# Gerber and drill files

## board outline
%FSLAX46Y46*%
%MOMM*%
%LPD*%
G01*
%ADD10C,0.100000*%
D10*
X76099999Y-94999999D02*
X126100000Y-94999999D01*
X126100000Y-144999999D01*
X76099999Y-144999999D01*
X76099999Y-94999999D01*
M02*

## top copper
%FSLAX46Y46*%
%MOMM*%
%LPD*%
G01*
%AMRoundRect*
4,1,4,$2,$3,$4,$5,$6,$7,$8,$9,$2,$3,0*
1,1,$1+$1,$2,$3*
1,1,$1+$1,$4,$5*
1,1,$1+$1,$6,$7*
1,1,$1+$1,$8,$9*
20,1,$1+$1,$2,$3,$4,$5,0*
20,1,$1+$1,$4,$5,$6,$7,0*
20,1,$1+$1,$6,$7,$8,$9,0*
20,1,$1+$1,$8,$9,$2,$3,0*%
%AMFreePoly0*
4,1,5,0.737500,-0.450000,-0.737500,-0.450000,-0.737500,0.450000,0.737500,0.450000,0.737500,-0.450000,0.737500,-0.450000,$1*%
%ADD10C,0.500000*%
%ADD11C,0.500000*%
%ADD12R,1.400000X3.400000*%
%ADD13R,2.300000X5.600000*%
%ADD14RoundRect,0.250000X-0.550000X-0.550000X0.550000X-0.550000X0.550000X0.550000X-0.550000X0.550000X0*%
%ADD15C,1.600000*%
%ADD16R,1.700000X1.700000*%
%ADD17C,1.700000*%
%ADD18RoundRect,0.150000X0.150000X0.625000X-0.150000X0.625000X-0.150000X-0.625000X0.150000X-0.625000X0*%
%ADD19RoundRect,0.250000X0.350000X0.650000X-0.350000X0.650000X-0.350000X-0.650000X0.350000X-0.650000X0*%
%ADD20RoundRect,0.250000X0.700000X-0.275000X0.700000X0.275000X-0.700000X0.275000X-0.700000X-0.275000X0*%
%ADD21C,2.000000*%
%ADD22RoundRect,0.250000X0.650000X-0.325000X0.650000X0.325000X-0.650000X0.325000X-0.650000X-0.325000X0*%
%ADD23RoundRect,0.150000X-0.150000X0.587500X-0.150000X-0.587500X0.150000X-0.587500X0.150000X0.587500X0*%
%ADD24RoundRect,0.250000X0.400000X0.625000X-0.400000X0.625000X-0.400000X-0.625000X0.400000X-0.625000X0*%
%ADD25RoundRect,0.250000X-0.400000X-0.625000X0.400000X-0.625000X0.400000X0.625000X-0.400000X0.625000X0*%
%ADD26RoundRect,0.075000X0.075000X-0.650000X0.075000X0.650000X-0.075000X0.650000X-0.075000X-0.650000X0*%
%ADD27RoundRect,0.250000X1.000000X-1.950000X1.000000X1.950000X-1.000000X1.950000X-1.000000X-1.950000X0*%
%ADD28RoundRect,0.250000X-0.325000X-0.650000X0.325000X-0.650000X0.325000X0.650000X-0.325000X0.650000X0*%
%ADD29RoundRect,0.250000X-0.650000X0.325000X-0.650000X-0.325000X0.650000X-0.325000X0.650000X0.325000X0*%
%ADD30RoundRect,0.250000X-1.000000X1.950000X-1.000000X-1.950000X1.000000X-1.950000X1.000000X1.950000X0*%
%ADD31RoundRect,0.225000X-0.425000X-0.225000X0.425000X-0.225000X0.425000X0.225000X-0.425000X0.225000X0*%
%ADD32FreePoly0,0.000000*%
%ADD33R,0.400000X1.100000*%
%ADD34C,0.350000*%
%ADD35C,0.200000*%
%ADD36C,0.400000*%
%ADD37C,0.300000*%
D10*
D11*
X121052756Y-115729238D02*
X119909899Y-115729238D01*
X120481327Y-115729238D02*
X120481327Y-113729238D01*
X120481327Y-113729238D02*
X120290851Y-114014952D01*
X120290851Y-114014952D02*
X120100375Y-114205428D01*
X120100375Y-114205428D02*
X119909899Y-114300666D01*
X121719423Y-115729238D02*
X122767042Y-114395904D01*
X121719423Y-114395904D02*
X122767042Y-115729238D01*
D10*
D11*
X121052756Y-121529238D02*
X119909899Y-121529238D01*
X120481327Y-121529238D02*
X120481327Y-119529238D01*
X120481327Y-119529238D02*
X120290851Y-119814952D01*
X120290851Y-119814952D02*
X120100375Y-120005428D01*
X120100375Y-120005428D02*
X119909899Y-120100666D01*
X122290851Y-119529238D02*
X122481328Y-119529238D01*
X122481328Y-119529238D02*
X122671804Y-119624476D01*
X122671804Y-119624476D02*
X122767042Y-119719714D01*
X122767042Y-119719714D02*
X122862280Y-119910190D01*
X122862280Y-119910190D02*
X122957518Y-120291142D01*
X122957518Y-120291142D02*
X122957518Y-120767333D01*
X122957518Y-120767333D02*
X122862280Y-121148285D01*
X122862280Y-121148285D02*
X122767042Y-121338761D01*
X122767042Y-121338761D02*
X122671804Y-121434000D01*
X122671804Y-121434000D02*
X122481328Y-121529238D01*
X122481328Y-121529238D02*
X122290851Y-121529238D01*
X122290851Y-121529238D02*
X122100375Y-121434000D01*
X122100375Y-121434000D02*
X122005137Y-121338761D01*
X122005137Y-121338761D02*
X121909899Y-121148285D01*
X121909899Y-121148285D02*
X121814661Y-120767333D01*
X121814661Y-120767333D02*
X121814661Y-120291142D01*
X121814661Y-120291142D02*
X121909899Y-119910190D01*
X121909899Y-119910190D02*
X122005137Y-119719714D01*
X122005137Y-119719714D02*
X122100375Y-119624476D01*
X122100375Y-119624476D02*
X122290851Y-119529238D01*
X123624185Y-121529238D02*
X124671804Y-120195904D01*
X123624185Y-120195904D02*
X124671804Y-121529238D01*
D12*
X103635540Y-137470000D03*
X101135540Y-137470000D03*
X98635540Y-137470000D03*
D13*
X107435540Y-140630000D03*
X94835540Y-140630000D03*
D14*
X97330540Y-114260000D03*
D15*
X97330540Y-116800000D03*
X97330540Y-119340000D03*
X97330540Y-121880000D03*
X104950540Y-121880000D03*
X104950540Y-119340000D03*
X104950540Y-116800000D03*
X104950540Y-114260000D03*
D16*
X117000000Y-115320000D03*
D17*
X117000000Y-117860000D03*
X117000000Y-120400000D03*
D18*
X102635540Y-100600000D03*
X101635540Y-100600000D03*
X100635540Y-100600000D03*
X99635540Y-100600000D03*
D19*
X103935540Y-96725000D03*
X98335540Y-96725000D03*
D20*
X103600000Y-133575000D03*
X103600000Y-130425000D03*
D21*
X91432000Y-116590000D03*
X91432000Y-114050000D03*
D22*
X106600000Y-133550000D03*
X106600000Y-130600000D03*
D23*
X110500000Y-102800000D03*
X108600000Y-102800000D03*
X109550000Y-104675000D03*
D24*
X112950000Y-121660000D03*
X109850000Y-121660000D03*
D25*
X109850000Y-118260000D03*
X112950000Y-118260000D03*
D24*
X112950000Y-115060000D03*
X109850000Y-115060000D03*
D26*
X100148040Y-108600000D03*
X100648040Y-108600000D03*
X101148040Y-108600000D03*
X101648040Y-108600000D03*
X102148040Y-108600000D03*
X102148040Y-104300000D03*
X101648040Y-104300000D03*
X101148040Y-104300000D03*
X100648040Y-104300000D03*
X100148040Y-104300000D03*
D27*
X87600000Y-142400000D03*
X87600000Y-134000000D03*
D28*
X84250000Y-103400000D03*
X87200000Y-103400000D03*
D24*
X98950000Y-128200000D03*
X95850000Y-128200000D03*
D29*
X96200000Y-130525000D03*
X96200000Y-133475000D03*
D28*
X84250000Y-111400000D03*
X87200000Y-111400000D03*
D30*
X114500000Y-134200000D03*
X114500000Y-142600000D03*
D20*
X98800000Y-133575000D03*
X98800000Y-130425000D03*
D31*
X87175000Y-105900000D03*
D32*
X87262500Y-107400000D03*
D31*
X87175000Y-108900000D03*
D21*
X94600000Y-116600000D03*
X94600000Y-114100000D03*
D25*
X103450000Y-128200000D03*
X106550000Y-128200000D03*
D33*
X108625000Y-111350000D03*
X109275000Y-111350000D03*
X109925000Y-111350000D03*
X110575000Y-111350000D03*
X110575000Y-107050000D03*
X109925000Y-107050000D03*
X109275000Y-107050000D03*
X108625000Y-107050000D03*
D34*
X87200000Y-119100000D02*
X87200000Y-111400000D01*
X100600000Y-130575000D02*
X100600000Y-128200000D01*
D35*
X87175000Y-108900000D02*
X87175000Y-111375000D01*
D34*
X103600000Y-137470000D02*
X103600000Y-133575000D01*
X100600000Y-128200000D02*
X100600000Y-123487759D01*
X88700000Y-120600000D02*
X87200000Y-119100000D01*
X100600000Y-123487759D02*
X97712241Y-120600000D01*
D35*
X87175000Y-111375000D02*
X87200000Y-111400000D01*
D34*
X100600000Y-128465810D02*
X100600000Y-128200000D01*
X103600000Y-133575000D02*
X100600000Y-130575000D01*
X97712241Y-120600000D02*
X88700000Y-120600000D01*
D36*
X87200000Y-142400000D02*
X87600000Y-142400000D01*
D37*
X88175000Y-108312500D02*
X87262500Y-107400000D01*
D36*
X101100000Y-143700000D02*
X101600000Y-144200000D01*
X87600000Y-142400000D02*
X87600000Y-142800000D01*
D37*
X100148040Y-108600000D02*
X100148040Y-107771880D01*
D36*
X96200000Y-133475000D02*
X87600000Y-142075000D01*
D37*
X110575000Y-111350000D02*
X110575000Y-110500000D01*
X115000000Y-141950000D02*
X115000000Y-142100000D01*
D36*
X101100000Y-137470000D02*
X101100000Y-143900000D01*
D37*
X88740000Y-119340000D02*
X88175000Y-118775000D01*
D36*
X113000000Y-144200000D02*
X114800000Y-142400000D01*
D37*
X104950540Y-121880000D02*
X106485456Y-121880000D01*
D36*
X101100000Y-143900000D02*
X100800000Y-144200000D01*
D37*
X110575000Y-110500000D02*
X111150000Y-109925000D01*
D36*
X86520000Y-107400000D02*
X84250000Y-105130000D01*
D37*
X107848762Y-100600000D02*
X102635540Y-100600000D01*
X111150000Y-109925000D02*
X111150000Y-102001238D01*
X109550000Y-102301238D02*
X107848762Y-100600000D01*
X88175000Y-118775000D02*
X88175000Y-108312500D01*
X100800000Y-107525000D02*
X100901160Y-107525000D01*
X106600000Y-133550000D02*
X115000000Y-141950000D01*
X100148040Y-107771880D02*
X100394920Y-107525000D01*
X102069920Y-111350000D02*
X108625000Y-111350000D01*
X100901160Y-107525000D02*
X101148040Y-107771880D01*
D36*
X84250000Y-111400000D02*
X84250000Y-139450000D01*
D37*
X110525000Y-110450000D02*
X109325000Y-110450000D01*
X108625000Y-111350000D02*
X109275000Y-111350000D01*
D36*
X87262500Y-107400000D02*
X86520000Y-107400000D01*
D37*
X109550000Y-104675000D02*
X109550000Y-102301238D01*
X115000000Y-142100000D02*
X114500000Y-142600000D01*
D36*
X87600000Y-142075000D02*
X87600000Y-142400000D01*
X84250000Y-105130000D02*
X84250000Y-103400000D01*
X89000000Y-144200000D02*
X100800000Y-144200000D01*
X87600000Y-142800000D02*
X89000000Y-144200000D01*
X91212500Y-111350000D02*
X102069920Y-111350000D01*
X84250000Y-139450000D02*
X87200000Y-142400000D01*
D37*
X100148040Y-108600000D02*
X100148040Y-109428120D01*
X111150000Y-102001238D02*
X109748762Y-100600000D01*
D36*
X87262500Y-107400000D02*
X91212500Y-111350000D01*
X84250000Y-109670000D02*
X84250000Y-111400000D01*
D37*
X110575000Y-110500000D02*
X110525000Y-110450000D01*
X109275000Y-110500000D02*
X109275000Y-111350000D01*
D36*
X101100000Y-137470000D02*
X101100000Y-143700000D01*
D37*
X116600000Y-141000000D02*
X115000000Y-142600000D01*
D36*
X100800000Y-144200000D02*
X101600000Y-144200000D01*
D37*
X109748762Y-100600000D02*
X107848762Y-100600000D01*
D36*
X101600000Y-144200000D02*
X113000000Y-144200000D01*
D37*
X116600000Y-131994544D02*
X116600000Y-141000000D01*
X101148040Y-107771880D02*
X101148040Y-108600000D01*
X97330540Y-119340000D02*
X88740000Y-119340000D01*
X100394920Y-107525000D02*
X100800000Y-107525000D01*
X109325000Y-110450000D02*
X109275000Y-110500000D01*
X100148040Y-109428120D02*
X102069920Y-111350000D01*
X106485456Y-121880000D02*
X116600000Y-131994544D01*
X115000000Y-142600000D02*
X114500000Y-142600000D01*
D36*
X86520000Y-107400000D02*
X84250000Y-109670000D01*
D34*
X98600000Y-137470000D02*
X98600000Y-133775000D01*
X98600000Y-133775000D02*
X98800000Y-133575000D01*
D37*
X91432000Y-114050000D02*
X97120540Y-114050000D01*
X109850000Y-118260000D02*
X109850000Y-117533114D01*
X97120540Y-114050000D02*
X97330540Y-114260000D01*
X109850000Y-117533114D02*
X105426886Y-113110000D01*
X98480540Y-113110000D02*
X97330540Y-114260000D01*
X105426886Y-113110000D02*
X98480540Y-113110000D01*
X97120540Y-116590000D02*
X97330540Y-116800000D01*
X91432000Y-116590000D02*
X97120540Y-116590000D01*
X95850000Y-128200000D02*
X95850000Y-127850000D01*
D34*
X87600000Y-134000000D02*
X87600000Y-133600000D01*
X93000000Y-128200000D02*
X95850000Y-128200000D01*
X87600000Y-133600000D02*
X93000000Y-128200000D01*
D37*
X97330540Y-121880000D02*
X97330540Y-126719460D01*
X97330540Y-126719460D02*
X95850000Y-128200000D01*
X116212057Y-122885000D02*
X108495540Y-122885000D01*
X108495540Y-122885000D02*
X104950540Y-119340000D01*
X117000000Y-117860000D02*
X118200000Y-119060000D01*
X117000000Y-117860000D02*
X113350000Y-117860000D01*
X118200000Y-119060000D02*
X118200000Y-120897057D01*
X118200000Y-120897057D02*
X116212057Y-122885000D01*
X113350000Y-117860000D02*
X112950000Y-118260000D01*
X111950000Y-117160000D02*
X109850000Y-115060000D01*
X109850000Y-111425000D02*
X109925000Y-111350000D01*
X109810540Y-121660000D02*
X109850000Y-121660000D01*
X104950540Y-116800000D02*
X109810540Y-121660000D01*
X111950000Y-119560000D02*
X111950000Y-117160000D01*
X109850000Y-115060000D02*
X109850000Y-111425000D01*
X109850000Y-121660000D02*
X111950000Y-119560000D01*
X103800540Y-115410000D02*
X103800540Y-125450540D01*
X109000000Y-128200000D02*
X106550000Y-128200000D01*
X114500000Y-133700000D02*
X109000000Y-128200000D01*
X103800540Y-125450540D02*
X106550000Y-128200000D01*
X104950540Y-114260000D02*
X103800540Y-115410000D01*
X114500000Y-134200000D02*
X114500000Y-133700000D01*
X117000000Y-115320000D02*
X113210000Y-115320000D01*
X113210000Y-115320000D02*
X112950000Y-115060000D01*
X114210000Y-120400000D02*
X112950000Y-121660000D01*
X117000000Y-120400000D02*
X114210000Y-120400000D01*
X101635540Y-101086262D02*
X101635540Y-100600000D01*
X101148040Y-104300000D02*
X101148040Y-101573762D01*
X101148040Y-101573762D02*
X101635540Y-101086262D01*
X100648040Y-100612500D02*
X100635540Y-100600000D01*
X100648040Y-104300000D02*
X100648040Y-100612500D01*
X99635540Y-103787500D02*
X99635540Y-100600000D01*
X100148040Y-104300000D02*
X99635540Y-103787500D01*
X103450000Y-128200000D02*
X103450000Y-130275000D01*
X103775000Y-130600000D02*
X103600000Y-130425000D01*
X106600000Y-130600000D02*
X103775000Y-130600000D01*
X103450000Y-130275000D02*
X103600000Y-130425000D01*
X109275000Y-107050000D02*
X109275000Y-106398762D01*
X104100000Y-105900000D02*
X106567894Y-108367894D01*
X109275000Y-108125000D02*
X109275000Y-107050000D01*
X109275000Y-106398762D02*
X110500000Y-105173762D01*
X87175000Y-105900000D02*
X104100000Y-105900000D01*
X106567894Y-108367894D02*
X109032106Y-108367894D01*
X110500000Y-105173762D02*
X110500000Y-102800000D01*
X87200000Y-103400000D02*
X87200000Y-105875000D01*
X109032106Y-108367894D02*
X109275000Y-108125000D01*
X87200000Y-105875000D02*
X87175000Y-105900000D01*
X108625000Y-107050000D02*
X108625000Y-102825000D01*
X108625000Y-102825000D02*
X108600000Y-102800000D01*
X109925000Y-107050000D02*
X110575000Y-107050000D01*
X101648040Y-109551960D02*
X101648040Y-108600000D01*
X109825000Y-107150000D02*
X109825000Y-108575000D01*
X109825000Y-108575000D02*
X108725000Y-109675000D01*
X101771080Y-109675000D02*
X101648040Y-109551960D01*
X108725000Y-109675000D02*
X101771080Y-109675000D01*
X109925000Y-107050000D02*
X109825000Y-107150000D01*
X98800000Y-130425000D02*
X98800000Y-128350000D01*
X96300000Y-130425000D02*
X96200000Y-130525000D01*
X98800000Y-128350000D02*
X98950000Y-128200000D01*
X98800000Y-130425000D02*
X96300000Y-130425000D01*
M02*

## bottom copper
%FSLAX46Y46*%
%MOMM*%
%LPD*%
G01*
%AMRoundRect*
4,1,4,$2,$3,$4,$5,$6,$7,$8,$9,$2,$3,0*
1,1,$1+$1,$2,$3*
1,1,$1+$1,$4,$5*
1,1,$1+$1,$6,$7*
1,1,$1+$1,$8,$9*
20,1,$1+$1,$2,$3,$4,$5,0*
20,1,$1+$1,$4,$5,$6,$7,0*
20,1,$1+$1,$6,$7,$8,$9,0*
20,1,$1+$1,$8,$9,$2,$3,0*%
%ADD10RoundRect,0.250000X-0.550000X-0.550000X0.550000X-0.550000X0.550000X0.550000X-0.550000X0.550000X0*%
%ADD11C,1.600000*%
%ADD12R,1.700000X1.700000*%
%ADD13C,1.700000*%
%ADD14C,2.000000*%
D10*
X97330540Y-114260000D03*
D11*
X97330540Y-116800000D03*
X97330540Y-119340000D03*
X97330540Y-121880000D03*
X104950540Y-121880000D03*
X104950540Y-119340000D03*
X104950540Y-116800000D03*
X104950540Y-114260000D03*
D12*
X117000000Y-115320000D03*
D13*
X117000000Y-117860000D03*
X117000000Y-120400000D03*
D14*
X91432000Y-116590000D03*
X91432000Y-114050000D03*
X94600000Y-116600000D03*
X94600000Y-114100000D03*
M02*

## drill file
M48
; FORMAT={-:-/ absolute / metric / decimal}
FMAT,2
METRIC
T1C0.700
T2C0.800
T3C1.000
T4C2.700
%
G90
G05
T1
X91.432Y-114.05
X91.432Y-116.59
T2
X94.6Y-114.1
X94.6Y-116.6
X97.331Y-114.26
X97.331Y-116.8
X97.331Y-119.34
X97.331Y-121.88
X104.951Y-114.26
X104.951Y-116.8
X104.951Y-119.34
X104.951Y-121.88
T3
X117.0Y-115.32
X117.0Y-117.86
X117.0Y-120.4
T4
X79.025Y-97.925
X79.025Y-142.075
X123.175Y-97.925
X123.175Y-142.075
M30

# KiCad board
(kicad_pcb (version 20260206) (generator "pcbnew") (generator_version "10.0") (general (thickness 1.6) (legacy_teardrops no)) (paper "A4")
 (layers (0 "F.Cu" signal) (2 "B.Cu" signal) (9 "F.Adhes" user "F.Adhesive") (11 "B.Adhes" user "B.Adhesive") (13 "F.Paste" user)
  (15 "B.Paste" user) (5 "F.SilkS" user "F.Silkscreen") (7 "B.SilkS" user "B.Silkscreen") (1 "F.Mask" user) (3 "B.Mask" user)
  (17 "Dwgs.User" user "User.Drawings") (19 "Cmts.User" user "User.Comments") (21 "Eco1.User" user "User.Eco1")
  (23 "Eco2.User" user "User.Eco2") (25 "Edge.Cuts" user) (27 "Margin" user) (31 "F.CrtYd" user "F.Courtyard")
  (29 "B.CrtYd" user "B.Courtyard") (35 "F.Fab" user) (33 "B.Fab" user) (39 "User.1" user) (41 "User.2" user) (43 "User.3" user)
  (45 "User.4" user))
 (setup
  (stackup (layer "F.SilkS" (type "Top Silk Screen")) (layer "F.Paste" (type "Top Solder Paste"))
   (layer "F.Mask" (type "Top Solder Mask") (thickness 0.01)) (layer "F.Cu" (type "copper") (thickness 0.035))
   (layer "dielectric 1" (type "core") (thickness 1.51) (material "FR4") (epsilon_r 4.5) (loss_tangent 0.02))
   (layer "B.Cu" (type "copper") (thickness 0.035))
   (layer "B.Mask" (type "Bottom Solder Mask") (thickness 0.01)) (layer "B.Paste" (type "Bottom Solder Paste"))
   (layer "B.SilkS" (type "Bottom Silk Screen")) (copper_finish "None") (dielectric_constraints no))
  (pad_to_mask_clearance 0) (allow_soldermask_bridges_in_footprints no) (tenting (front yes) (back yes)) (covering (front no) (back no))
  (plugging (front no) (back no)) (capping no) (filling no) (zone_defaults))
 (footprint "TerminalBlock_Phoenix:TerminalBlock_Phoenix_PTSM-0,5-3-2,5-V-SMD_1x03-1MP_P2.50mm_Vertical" (layer "F.Cu")
  (at 101.13554 139.6 180)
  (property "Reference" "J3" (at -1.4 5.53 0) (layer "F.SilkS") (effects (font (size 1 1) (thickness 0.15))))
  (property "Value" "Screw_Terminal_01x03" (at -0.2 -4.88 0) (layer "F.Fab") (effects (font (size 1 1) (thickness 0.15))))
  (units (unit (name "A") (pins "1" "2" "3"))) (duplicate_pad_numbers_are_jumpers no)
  (pad "1" smd rect (at -2.5 2.13) (size 1.4 3.4) (layers "F.Cu" "F.Mask" "F.Paste") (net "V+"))
  (pad "2" smd rect (at 0 2.13) (size 1.4 3.4) (layers "F.Cu" "F.Mask" "F.Paste") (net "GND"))
  (pad "3" smd rect (at 2.5 2.13) (size 1.4 3.4) (layers "F.Cu" "F.Mask" "F.Paste") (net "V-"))
  (pad "MP" smd rect (at -6.3 -1.03) (size 2.3 5.6) (layers "F.Cu" "F.Mask" "F.Paste"))
  (pad "MP" smd rect (at 6.3 -1.03) (size 2.3 5.6) (layers "F.Cu" "F.Mask" "F.Paste")))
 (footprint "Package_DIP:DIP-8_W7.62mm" (layer "F.Cu") (at 97.33054 114.26)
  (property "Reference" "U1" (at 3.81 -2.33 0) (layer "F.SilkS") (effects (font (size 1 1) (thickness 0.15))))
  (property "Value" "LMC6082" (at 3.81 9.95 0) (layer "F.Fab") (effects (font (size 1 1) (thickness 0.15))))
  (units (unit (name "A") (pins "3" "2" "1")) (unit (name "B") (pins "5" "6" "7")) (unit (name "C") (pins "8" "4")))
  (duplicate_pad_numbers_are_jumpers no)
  (pad "1" thru_hole roundrect (at 0 0) (size 1.6 1.6) (drill 0.8) (layers "*.Cu" "*.Mask") (remove_unused_layers no)
   (roundrect_rratio 0.15625) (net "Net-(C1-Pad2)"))
  (pad "2" thru_hole circle (at 0 2.54) (size 1.6 1.6) (drill 0.8) (layers "*.Cu" "*.Mask") (remove_unused_layers no) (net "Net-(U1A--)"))
  (pad "3" thru_hole circle (at 0 5.08) (size 1.6 1.6) (drill 0.8) (layers "*.Cu" "*.Mask") (remove_unused_layers no) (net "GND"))
  (pad "4" thru_hole circle (at 0 7.62) (size 1.6 1.6) (drill 0.8) (layers "*.Cu" "*.Mask") (remove_unused_layers no) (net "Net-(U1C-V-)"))
  (pad "5" thru_hole circle (at 7.62 7.62) (size 1.6 1.6) (drill 0.8) (layers "*.Cu" "*.Mask") (remove_unused_layers no) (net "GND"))
  (pad "6" thru_hole circle (at 7.62 5.08) (size 1.6 1.6) (drill 0.8) (layers "*.Cu" "*.Mask") (remove_unused_layers no)
   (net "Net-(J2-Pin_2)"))
  (pad "7" thru_hole circle (at 7.62 2.54) (size 1.6 1.6) (drill 0.8) (layers "*.Cu" "*.Mask") (remove_unused_layers no) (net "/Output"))
  (pad "8" thru_hole circle (at 7.62 0) (size 1.6 1.6) (drill 0.8) (layers "*.Cu" "*.Mask") (remove_unused_layers no) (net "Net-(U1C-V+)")))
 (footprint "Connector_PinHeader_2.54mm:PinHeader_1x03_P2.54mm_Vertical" (layer "F.Cu") (at 117 115.32)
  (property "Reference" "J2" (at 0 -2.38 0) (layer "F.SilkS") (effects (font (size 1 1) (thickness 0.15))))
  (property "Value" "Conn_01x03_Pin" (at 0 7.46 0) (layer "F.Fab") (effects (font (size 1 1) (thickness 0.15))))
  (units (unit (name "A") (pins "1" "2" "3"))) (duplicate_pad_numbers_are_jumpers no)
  (pad "1" thru_hole rect (at 0 0) (size 1.7 1.7) (drill 1) (layers "*.Cu" "*.Mask") (remove_unused_layers no) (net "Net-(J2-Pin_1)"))
  (pad "2" thru_hole circle (at 0 2.54) (size 1.7 1.7) (drill 1) (layers "*.Cu" "*.Mask") (remove_unused_layers no) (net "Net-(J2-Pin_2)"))
  (pad "3" thru_hole circle (at 0 5.08) (size 1.7 1.7) (drill 1) (layers "*.Cu" "*.Mask") (remove_unused_layers no) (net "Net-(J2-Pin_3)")))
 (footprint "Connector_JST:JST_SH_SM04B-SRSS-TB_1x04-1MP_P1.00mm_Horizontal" (layer "F.Cu") (at 101.13554 98.6 180)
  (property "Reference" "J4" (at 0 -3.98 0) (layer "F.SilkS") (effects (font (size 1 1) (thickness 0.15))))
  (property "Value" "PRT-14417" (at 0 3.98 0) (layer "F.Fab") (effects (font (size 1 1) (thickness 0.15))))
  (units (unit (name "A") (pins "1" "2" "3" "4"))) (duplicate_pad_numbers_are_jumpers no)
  (pad "1" smd roundrect (at -1.5 -2 180) (size 0.6 1.55) (layers "F.Cu" "F.Mask" "F.Paste") (roundrect_rratio 0.25) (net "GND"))
  (pad "2" smd roundrect (at -0.5 -2 180) (size 0.6 1.55) (layers "F.Cu" "F.Mask" "F.Paste") (roundrect_rratio 0.25) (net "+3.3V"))
  (pad "3" smd roundrect (at 0.5 -2 180) (size 0.6 1.55) (layers "F.Cu" "F.Mask" "F.Paste") (roundrect_rratio 0.25) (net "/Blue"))
  (pad "4" smd roundrect (at 1.5 -2 180) (size 0.6 1.55) (layers "F.Cu" "F.Mask" "F.Paste") (roundrect_rratio 0.25) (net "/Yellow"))
  (pad "MP" smd roundrect (at -2.8 1.875 180) (size 1.2 1.8) (layers "F.Cu" "F.Mask" "F.Paste") (roundrect_rratio 0.208333))
  (pad "MP" smd roundrect (at 2.8 1.875 180) (size 1.2 1.8) (layers "F.Cu" "F.Mask" "F.Paste") (roundrect_rratio 0.208333)))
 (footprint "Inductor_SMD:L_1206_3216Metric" (layer "F.Cu") (at 103.6 132 90)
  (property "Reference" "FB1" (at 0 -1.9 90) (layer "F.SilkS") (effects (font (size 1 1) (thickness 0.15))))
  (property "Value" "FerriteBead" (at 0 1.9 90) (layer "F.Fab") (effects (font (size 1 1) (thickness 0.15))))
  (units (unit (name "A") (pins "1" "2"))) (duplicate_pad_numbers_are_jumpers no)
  (pad "1" smd roundrect (at -1.575 0 90) (size 1.05 1.9) (layers "F.Cu" "F.Mask" "F.Paste") (roundrect_rratio 0.238095) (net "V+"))
  (pad "2" smd roundrect (at 1.575 0 90) (size 1.05 1.9) (layers "F.Cu" "F.Mask" "F.Paste") (roundrect_rratio 0.238095)
   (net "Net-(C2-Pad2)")))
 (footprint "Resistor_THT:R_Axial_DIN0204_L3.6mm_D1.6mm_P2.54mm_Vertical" (layer "F.Cu") (at 91.432 116.59 90)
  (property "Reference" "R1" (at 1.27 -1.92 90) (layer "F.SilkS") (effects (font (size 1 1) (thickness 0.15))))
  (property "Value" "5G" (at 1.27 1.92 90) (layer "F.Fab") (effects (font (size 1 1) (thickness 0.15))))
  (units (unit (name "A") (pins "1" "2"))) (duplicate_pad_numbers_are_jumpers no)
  (pad "1" thru_hole circle (at 0 0 90) (size 2 2) (drill 0.7) (layers "*.Cu" "*.Mask") (remove_unused_layers no) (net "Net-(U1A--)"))
  (pad "2" thru_hole circle (at 2.54 0 90) (size 2 2) (drill 0.7) (layers "*.Cu" "*.Mask") (remove_unused_layers no) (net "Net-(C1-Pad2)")))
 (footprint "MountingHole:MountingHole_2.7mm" (layer "F.Cu") (at 79.024999 142.074999)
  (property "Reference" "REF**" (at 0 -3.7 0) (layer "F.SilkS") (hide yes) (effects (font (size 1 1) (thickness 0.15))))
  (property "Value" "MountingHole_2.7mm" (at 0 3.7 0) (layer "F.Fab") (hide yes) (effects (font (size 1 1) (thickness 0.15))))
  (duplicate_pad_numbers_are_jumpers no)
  (pad "" np_thru_hole circle (at 0 0) (size 2.7 2.7) (drill 2.7) (layers "*.Cu" "*.Mask")))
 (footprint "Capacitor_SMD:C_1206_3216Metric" (layer "F.Cu") (at 106.6 132.075 90)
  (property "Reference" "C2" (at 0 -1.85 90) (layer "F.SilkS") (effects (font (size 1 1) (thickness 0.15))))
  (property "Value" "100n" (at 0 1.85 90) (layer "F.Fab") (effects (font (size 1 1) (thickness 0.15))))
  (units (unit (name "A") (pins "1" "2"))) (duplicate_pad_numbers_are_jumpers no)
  (pad "1" smd roundrect (at -1.475 0 90) (size 1.15 1.8) (layers "F.Cu" "F.Mask" "F.Paste") (roundrect_rratio 0.217391) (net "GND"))
  (pad "2" smd roundrect (at 1.475 0 90) (size 1.15 1.8) (layers "F.Cu" "F.Mask" "F.Paste") (roundrect_rratio 0.217391)
   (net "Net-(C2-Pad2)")))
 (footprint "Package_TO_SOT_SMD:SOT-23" (layer "F.Cu") (at 109.55 103.7375 -90)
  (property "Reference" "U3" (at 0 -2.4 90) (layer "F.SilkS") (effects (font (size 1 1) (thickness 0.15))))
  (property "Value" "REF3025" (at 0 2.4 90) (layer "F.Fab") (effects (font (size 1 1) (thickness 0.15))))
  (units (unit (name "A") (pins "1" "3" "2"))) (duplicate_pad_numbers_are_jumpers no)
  (pad "1" smd roundrect (at -0.9375 -0.95 270) (size 1.475 0.6) (layers "F.Cu" "F.Mask" "F.Paste") (roundrect_rratio 0.25) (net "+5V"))
  (pad "2" smd roundrect (at -0.9375 0.95 270) (size 1.475 0.6) (layers "F.Cu" "F.Mask" "F.Paste") (roundrect_rratio 0.25) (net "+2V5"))
  (pad "3" smd roundrect (at 0.9375 0 270) (size 1.475 0.6) (layers "F.Cu" "F.Mask" "F.Paste") (roundrect_rratio 0.25) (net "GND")))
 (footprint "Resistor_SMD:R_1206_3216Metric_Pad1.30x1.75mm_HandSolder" (layer "F.Cu") (at 111.4 121.66 180)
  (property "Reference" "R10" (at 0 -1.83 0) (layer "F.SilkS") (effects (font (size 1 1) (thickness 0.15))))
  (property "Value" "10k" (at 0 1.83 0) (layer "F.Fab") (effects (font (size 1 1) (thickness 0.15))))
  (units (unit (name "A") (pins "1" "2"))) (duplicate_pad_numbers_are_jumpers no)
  (pad "1" smd roundrect (at -1.55 0 180) (size 1.3 1.75) (layers "F.Cu" "F.Mask" "F.Paste") (roundrect_rratio 0.192308)
   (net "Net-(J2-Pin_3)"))
  (pad "2" smd roundrect (at 1.55 0 180) (size 1.3 1.75) (layers "F.Cu" "F.Mask" "F.Paste") (roundrect_rratio 0.192308) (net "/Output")))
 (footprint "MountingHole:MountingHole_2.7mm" (layer "F.Cu") (at 123.175 142.074999)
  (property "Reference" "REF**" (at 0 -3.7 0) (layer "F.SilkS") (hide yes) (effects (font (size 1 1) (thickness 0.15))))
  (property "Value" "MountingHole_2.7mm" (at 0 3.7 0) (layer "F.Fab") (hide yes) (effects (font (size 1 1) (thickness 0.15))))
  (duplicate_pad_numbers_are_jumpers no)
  (pad "" np_thru_hole circle (at 0 0) (size 2.7 2.7) (drill 2.7) (layers "*.Cu" "*.Mask")))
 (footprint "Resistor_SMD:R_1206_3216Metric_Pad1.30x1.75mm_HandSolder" (layer "F.Cu") (at 111.4 118.26)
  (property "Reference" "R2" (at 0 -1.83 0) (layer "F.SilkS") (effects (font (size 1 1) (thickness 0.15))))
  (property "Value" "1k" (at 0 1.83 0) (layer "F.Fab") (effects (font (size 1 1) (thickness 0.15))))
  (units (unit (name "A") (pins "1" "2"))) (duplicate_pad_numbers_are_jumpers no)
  (pad "1" smd roundrect (at -1.55 0) (size 1.3 1.75) (layers "F.Cu" "F.Mask" "F.Paste") (roundrect_rratio 0.192308) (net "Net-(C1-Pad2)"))
  (pad "2" smd roundrect (at 1.55 0) (size 1.3 1.75) (layers "F.Cu" "F.Mask" "F.Paste") (roundrect_rratio 0.192308) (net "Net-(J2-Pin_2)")))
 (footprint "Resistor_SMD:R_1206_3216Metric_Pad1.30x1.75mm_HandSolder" (layer "F.Cu") (at 111.4 115.06 180)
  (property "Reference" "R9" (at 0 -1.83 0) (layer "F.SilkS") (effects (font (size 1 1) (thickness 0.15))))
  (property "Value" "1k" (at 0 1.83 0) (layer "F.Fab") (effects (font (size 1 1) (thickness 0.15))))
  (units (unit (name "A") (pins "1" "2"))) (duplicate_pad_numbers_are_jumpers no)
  (pad "1" smd roundrect (at -1.55 0 180) (size 1.3 1.75) (layers "F.Cu" "F.Mask" "F.Paste") (roundrect_rratio 0.192308)
   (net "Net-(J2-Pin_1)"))
  (pad "2" smd roundrect (at 1.55 0 180) (size 1.3 1.75) (layers "F.Cu" "F.Mask" "F.Paste") (roundrect_rratio 0.192308) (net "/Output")))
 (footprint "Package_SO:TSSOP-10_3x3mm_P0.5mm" (layer "F.Cu") (at 101.14804 106.45 90)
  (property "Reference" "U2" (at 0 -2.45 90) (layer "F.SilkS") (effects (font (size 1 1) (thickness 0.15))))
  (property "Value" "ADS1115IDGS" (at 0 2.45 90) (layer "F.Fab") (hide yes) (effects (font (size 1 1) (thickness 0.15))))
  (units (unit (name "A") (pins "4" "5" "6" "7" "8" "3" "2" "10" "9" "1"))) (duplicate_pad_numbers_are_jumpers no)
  (pad "1" smd roundrect (at -2.15 -1 90) (size 1.45 0.3) (layers "F.Cu" "F.Mask" "F.Paste") (roundrect_rratio 0.25) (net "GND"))
  (pad "2" smd roundrect (at -2.15 -0.5 90) (size 1.45 0.3) (layers "F.Cu" "F.Mask" "F.Paste") (roundrect_rratio 0.25)
   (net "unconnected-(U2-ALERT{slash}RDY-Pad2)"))
  (pad "3" smd roundrect (at -2.15 0 90) (size 1.45 0.3) (layers "F.Cu" "F.Mask" "F.Paste") (roundrect_rratio 0.25) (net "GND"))
  (pad "4" smd roundrect (at -2.15 0.5 90) (size 1.45 0.3) (layers "F.Cu" "F.Mask" "F.Paste") (roundrect_rratio 0.25) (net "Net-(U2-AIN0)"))
  (pad "5" smd roundrect (at -2.15 1 90) (size 1.45 0.3) (layers "F.Cu" "F.Mask" "F.Paste") (roundrect_rratio 0.25)
   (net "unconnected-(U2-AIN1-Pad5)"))
  (pad "6" smd roundrect (at 2.15 1 90) (size 1.45 0.3) (layers "F.Cu" "F.Mask" "F.Paste") (roundrect_rratio 0.25)
   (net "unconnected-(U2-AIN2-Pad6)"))
  (pad "7" smd roundrect (at 2.15 0.5 90) (size 1.45 0.3) (layers "F.Cu" "F.Mask" "F.Paste") (roundrect_rratio 0.25)
   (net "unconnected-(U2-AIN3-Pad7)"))
  (pad "8" smd roundrect (at 2.15 0 90) (size 1.45 0.3) (layers "F.Cu" "F.Mask" "F.Paste") (roundrect_rratio 0.25) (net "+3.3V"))
  (pad "9" smd roundrect (at 2.15 -0.5 90) (size 1.45 0.3) (layers "F.Cu" "F.Mask" "F.Paste") (roundrect_rratio 0.25) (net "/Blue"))
  (pad "10" smd roundrect (at 2.15 -1 90) (size 1.45 0.3) (layers "F.Cu" "F.Mask" "F.Paste") (roundrect_rratio 0.25) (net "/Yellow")))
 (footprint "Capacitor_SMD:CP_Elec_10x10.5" (layer "F.Cu") (at 87.6 138.2 90)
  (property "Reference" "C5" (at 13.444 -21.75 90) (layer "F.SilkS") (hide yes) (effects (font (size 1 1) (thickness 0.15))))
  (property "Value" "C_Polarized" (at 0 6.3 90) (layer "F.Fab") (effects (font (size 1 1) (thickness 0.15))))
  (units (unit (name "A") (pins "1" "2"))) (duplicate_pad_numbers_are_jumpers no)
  (pad "1" smd roundrect (at -4.2 0 90) (size 4.4 2.5) (layers "F.Cu" "F.Mask" "F.Paste") (roundrect_rratio 0.1) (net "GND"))
  (pad "2" smd roundrect (at 4.2 0 90) (size 4.4 2.5) (layers "F.Cu" "F.Mask" "F.Paste") (roundrect_rratio 0.1) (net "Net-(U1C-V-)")))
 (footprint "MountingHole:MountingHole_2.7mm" (layer "F.Cu") (at 123.175 97.924999)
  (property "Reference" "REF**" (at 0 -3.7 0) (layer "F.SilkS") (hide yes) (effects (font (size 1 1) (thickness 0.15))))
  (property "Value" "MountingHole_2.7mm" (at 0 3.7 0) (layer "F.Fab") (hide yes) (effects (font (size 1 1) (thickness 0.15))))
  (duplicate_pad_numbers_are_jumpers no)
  (pad "" np_thru_hole circle (at 0 0) (size 2.7 2.7) (drill 2.7) (layers "*.Cu" "*.Mask")))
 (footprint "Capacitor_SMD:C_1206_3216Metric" (layer "F.Cu") (at 85.725 103.4)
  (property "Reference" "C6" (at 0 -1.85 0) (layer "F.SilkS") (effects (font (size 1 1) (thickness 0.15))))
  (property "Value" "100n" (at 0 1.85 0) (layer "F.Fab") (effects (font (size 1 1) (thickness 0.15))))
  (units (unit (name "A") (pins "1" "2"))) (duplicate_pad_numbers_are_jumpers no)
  (pad "1" smd roundrect (at -1.475 0) (size 1.15 1.8) (layers "F.Cu" "F.Mask" "F.Paste") (roundrect_rratio 0.217391) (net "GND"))
  (pad "2" smd roundrect (at 1.475 0) (size 1.15 1.8) (layers "F.Cu" "F.Mask" "F.Paste") (roundrect_rratio 0.217391) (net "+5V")))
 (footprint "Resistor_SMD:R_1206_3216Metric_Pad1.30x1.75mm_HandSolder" (layer "F.Cu") (at 97.4 128.2 180)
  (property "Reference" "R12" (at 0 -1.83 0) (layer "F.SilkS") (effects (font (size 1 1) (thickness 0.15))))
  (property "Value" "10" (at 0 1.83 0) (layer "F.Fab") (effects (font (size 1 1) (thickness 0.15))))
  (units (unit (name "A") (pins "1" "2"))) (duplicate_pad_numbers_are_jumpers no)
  (pad "1" smd roundrect (at -1.55 0 180) (size 1.3 1.75) (layers "F.Cu" "F.Mask" "F.Paste") (roundrect_rratio 0.192308)
   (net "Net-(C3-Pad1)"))
  (pad "2" smd roundrect (at 1.55 0 180) (size 1.3 1.75) (layers "F.Cu" "F.Mask" "F.Paste") (roundrect_rratio 0.192308) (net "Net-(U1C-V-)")))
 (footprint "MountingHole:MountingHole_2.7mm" (layer "F.Cu") (at 79.024999 97.924999)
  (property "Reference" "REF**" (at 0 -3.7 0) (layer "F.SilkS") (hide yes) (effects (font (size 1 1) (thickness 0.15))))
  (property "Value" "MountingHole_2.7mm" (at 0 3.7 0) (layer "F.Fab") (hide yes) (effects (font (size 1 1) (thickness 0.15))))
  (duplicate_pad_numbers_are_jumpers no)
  (pad "" np_thru_hole circle (at 0 0) (size 2.7 2.7) (drill 2.7) (layers "*.Cu" "*.Mask")))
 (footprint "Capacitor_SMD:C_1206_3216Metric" (layer "F.Cu") (at 96.2 132 -90)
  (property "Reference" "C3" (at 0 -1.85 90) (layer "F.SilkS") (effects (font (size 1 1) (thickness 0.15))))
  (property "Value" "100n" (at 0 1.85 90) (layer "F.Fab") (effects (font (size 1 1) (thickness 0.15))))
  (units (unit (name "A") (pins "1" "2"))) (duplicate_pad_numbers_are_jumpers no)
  (pad "1" smd roundrect (at -1.475 0 270) (size 1.15 1.8) (layers "F.Cu" "F.Mask" "F.Paste") (roundrect_rratio 0.217391)
   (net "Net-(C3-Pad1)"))
  (pad "2" smd roundrect (at 1.475 0 270) (size 1.15 1.8) (layers "F.Cu" "F.Mask" "F.Paste") (roundrect_rratio 0.217391) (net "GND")))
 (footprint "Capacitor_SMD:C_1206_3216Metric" (layer "F.Cu") (at 85.725 111.4)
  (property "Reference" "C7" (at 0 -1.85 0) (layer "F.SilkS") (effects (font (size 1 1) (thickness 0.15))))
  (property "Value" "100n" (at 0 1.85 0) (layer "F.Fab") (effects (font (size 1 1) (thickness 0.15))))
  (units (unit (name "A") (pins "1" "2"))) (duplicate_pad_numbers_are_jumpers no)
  (pad "1" smd roundrect (at -1.475 0) (size 1.15 1.8) (layers "F.Cu" "F.Mask" "F.Paste") (roundrect_rratio 0.217391) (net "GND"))
  (pad "2" smd roundrect (at 1.475 0) (size 1.15 1.8) (layers "F.Cu" "F.Mask" "F.Paste") (roundrect_rratio 0.217391) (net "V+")))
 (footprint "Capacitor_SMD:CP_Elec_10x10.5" (layer "F.Cu") (at 114.5 138.4 -90)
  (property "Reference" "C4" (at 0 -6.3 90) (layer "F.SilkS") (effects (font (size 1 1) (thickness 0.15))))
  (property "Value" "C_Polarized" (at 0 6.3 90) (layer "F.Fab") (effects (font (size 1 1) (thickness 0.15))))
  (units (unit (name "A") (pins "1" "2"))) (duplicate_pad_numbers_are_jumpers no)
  (pad "1" smd roundrect (at -4.2 0 270) (size 4.4 2.5) (layers "F.Cu" "F.Mask" "F.Paste") (roundrect_rratio 0.1) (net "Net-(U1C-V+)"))
  (pad "2" smd roundrect (at 4.2 0 270) (size 4.4 2.5) (layers "F.Cu" "F.Mask" "F.Paste") (roundrect_rratio 0.1) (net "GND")))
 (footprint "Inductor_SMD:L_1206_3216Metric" (layer "F.Cu") (at 98.8 132 90)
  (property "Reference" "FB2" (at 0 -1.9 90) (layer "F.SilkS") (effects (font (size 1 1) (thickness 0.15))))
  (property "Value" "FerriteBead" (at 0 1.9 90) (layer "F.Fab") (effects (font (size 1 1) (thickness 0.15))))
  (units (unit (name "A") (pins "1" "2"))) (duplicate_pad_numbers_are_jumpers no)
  (pad "1" smd roundrect (at -1.575 0 90) (size 1.05 1.9) (layers "F.Cu" "F.Mask" "F.Paste") (roundrect_rratio 0.238095) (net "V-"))
  (pad "2" smd roundrect (at 1.575 0 90) (size 1.05 1.9) (layers "F.Cu" "F.Mask" "F.Paste") (roundrect_rratio 0.238095)
   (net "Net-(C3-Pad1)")))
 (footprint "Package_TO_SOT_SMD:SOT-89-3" (layer "F.Cu") (at 89.125 107.4)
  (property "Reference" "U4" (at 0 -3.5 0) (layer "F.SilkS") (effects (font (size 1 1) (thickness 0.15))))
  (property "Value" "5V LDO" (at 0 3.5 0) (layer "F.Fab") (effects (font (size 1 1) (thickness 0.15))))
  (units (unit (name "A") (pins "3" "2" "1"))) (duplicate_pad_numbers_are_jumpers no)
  (pad "1" smd roundrect (at -1.95 -1.5) (size 1.3 0.9) (layers "F.Cu" "F.Mask" "F.Paste") (roundrect_rratio 0.25) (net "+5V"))
  (pad "2" smd custom (at -1.8625 0) (size 1.475 0.9) (layers "F.Cu" "F.Mask" "F.Paste") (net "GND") (zone_connect 2)
   (thermal_bridge_angle 45) (options (clearance outline) (anchor rect)) (primitives))
  (pad "3" smd roundrect (at -1.95 1.5) (size 1.3 0.9) (layers "F.Cu" "F.Mask" "F.Paste") (roundrect_rratio 0.25) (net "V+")))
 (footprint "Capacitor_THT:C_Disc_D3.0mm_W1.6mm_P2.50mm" (layer "F.Cu") (at 94.6 116.6 90)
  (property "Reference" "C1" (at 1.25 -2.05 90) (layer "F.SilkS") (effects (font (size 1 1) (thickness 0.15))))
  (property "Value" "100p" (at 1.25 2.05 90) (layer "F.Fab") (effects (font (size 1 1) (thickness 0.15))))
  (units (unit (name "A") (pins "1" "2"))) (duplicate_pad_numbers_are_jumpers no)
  (pad "1" thru_hole circle (at 0 0 90) (size 2 2) (drill 0.8) (layers "*.Cu" "*.Mask") (remove_unused_layers no) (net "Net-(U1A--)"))
  (pad "2" thru_hole circle (at 2.5 0 90) (size 2 2) (drill 0.8) (layers "*.Cu" "*.Mask") (remove_unused_layers no) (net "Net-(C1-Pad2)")))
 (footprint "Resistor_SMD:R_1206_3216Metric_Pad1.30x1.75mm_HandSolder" (layer "F.Cu") (at 105 128.2)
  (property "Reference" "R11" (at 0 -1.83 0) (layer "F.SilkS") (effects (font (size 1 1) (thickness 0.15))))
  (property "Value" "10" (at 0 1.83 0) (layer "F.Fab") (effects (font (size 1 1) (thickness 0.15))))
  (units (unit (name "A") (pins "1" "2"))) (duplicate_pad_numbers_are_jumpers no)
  (pad "1" smd roundrect (at -1.55 0) (size 1.3 1.75) (layers "F.Cu" "F.Mask" "F.Paste") (roundrect_rratio 0.192308) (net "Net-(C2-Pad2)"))
  (pad "2" smd roundrect (at 1.55 0) (size 1.3 1.75) (layers "F.Cu" "F.Mask" "F.Paste") (roundrect_rratio 0.192308) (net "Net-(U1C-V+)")))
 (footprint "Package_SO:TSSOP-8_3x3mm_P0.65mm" (layer "F.Cu") (at 109.6 109.2 90)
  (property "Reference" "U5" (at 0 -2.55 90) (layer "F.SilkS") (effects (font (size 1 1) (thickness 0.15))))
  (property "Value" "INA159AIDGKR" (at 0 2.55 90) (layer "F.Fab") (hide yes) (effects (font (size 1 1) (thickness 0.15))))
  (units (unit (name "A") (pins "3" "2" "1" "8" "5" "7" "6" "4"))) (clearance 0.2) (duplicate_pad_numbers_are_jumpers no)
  (pad "1" smd rect (at -2.15 -0.975 90) (size 1.1 0.4) (layers "F.Cu" "F.Mask" "F.Paste") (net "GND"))
  (pad "2" smd rect (at -2.15 -0.325 90) (size 1.1 0.4) (layers "F.Cu" "F.Mask" "F.Paste") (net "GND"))
  (pad "3" smd rect (at -2.15 0.325 90) (size 1.1 0.4) (layers "F.Cu" "F.Mask" "F.Paste") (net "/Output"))
  (pad "4" smd rect (at -2.15 0.975 90) (size 1.1 0.4) (layers "F.Cu" "F.Mask" "F.Paste") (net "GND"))
  (pad "5" smd rect (at 2.15 0.975 90) (size 1.1 0.4) (layers "F.Cu" "F.Mask" "F.Paste") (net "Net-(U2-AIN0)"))
  (pad "6" smd rect (at 2.15 0.325 90) (size 1.1 0.4) (layers "F.Cu" "F.Mask" "F.Paste") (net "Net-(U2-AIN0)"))
  (pad "7" smd rect (at 2.15 -0.325 90) (size 1.1 0.4) (layers "F.Cu" "F.Mask" "F.Paste") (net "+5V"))
  (pad "8" smd rect (at 2.15 -0.975 90) (size 1.1 0.4) (layers "F.Cu" "F.Mask" "F.Paste") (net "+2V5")))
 (gr_rect (start 76.099999 94.999999) (end 126.1 144.999999) (stroke (width 0.1) (type solid)) (fill no) (layer "Edge.Cuts"))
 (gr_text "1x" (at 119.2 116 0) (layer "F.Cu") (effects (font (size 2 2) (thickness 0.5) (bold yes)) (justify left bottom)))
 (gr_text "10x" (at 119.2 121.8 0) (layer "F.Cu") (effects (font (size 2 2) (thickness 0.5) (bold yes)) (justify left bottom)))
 (segment (start 87.2 119.1) (end 87.2 111.4) (width 0.35) (layer "F.Cu") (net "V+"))
 (segment (start 100.6 130.575) (end 100.6 128.2) (width 0.35) (layer "F.Cu") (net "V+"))
 (segment (start 87.175 108.9) (end 87.175 111.375) (width 0.2) (layer "F.Cu") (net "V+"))
 (segment (start 103.6 137.47) (end 103.6 133.575) (width 0.35) (layer "F.Cu") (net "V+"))
 (segment (start 100.6 128.2) (end 100.6 123.487759) (width 0.35) (layer "F.Cu") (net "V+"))
 (segment (start 88.7 120.6) (end 87.2 119.1) (width 0.35) (layer "F.Cu") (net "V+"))
 (segment (start 100.6 123.487759) (end 97.712241 120.6) (width 0.35) (layer "F.Cu") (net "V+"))
 (segment (start 87.175 111.375) (end 87.2 111.4) (width 0.2) (layer "F.Cu") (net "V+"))
 (segment (start 100.6 128.46581) (end 100.6 128.2) (width 0.35) (layer "F.Cu") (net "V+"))
 (segment (start 103.6 133.575) (end 100.6 130.575) (width 0.35) (layer "F.Cu") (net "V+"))
 (segment (start 97.712241 120.6) (end 88.7 120.6) (width 0.35) (layer "F.Cu") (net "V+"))
 (segment (start 87.2 142.4) (end 87.6 142.4) (width 0.4) (layer "F.Cu") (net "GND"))
 (segment (start 88.175 108.3125) (end 87.2625 107.4) (width 0.3) (layer "F.Cu") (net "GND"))
 (segment (start 101.1 143.7) (end 101.6 144.2) (width 0.4) (layer "F.Cu") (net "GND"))
 (segment (start 87.6 142.4) (end 87.6 142.8) (width 0.4) (layer "F.Cu") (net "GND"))
 (segment (start 100.14804 108.6) (end 100.14804 107.77188) (width 0.3) (layer "F.Cu") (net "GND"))
 (segment (start 96.2 133.475) (end 87.6 142.075) (width 0.4) (layer "F.Cu") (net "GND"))
 (segment (start 110.575 111.35) (end 110.575 110.5) (width 0.3) (layer "F.Cu") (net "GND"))
 (segment (start 115 141.95) (end 115 142.1) (width 0.3) (layer "F.Cu") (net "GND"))
 (segment (start 101.1 137.47) (end 101.1 143.9) (width 0.4) (layer "F.Cu") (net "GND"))
 (segment (start 88.74 119.34) (end 88.175 118.775) (width 0.3) (layer "F.Cu") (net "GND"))
 (segment (start 113 144.2) (end 114.8 142.4) (width 0.4) (layer "F.Cu") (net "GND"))
 (segment (start 104.95054 121.88) (end 106.485456 121.88) (width 0.3) (layer "F.Cu") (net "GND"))
 (segment (start 101.1 143.9) (end 100.8 144.2) (width 0.4) (layer "F.Cu") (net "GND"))
 (segment (start 110.575 110.5) (end 111.15 109.925) (width 0.3) (layer "F.Cu") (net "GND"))
 (segment (start 86.52 107.4) (end 84.25 105.13) (width 0.4) (layer "F.Cu") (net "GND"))
 (segment (start 107.848762 100.6) (end 102.63554 100.6) (width 0.3) (layer "F.Cu") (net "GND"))
 (segment (start 111.15 109.925) (end 111.15 102.001238) (width 0.3) (layer "F.Cu") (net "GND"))
 (segment (start 109.55 102.301238) (end 107.848762 100.6) (width 0.3) (layer "F.Cu") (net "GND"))
 (segment (start 88.175 118.775) (end 88.175 108.3125) (width 0.3) (layer "F.Cu") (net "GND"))
 (segment (start 100.8 107.525) (end 100.90116 107.525) (width 0.3) (layer "F.Cu") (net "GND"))
 (segment (start 106.6 133.55) (end 115 141.95) (width 0.3) (layer "F.Cu") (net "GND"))
 (segment (start 100.14804 107.77188) (end 100.39492 107.525) (width 0.3) (layer "F.Cu") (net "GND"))
 (segment (start 102.06992 111.35) (end 108.625 111.35) (width 0.3) (layer "F.Cu") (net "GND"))
 (segment (start 100.90116 107.525) (end 101.14804 107.77188) (width 0.3) (layer "F.Cu") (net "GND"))
 (segment (start 84.25 111.4) (end 84.25 139.45) (width 0.4) (layer "F.Cu") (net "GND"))
 (segment (start 110.525 110.45) (end 109.325 110.45) (width 0.3) (layer "F.Cu") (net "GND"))
 (segment (start 108.625 111.35) (end 109.275 111.35) (width 0.3) (layer "F.Cu") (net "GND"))
 (segment (start 87.2625 107.4) (end 86.52 107.4) (width 0.4) (layer "F.Cu") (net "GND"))
 (segment (start 109.55 104.675) (end 109.55 102.301238) (width 0.3) (layer "F.Cu") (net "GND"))
 (segment (start 115 142.1) (end 114.5 142.6) (width 0.3) (layer "F.Cu") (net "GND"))
 (segment (start 87.6 142.075) (end 87.6 142.4) (width 0.4) (layer "F.Cu") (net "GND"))
 (segment (start 84.25 105.13) (end 84.25 103.4) (width 0.4) (layer "F.Cu") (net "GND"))
 (segment (start 89 144.2) (end 100.8 144.2) (width 0.4) (layer "F.Cu") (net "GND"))
 (segment (start 87.6 142.8) (end 89 144.2) (width 0.4) (layer "F.Cu") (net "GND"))
 (segment (start 91.2125 111.35) (end 102.06992 111.35) (width 0.4) (layer "F.Cu") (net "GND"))
 (segment (start 84.25 139.45) (end 87.2 142.4) (width 0.4) (layer "F.Cu") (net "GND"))
 (segment (start 100.14804 108.6) (end 100.14804 109.42812) (width 0.3) (layer "F.Cu") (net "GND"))
 (segment (start 111.15 102.001238) (end 109.748762 100.6) (width 0.3) (layer "F.Cu") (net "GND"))
 (segment (start 87.2625 107.4) (end 91.2125 111.35) (width 0.4) (layer "F.Cu") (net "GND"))
 (segment (start 84.25 109.67) (end 84.25 111.4) (width 0.4) (layer "F.Cu") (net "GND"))
 (segment (start 110.575 110.5) (end 110.525 110.45) (width 0.3) (layer "F.Cu") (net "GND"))
 (segment (start 109.275 110.5) (end 109.275 111.35) (width 0.3) (layer "F.Cu") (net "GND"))
 (segment (start 101.1 137.47) (end 101.1 143.7) (width 0.4) (layer "F.Cu") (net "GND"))
 (segment (start 116.6 141) (end 115 142.6) (width 0.3) (layer "F.Cu") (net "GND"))
 (segment (start 100.8 144.2) (end 101.6 144.2) (width 0.4) (layer "F.Cu") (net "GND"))
 (segment (start 109.748762 100.6) (end 107.848762 100.6) (width 0.3) (layer "F.Cu") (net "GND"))
 (segment (start 101.6 144.2) (end 113 144.2) (width 0.4) (layer "F.Cu") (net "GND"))
 (segment (start 116.6 131.994544) (end 116.6 141) (width 0.3) (layer "F.Cu") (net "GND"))
 (segment (start 101.14804 107.77188) (end 101.14804 108.6) (width 0.3) (layer "F.Cu") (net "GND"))
 (segment (start 97.33054 119.34) (end 88.74 119.34) (width 0.3) (layer "F.Cu") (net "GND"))
 (segment (start 100.39492 107.525) (end 100.8 107.525) (width 0.3) (layer "F.Cu") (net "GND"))
 (segment (start 109.325 110.45) (end 109.275 110.5) (width 0.3) (layer "F.Cu") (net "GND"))
 (segment (start 100.14804 109.42812) (end 102.06992 111.35) (width 0.3) (layer "F.Cu") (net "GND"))
 (segment (start 106.485456 121.88) (end 116.6 131.994544) (width 0.3) (layer "F.Cu") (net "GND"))
 (segment (start 115 142.6) (end 114.5 142.6) (width 0.3) (layer "F.Cu") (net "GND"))
 (segment (start 86.52 107.4) (end 84.25 109.67) (width 0.4) (layer "F.Cu") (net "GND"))
 (segment (start 98.6 137.47) (end 98.6 133.775) (width 0.35) (layer "F.Cu") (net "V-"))
 (segment (start 98.6 133.775) (end 98.8 133.575) (width 0.35) (layer "F.Cu") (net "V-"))
 (segment (start 91.432 114.05) (end 97.12054 114.05) (width 0.3) (layer "F.Cu") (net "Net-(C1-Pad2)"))
 (segment (start 109.85 118.26) (end 109.85 117.533114) (width 0.3) (layer "F.Cu") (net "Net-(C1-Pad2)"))
 (segment (start 97.12054 114.05) (end 97.33054 114.26) (width 0.3) (layer "F.Cu") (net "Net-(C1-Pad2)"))
 (segment (start 109.85 117.533114) (end 105.426886 113.11) (width 0.3) (layer "F.Cu") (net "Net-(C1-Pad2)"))
 (segment (start 98.48054 113.11) (end 97.33054 114.26) (width 0.3) (layer "F.Cu") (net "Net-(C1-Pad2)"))
 (segment (start 105.426886 113.11) (end 98.48054 113.11) (width 0.3) (layer "F.Cu") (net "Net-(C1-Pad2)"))
 (segment (start 97.12054 116.59) (end 97.33054 116.8) (width 0.3) (layer "F.Cu") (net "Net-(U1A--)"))
 (segment (start 91.432 116.59) (end 97.12054 116.59) (width 0.3) (layer "F.Cu") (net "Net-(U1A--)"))
 (segment (start 95.85 128.2) (end 95.85 127.85) (width 0.3) (layer "F.Cu") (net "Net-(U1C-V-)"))
 (segment (start 87.6 134) (end 87.6 133.6) (width 0.35) (layer "F.Cu") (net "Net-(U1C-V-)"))
 (segment (start 93 128.2) (end 95.85 128.2) (width 0.35) (layer "F.Cu") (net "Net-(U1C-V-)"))
 (segment (start 87.6 133.6) (end 93 128.2) (width 0.35) (layer "F.Cu") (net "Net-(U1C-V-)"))
 (segment (start 97.33054 121.88) (end 97.33054 126.71946) (width 0.3) (layer "F.Cu") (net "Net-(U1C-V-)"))
 (segment (start 97.33054 126.71946) (end 95.85 128.2) (width 0.3) (layer "F.Cu") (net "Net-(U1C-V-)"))
 (segment (start 116.212057 122.885) (end 108.49554 122.885) (width 0.3) (layer "F.Cu") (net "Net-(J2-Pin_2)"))
 (segment (start 108.49554 122.885) (end 104.95054 119.34) (width 0.3) (layer "F.Cu") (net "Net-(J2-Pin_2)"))
 (segment (start 117 117.86) (end 118.2 119.06) (width 0.3) (layer "F.Cu") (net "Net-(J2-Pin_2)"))
 (segment (start 117 117.86) (end 113.35 117.86) (width 0.3) (layer "F.Cu") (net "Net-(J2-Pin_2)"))
 (segment (start 118.2 119.06) (end 118.2 120.897057) (width 0.3) (layer "F.Cu") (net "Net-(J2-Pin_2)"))
 (segment (start 118.2 120.897057) (end 116.212057 122.885) (width 0.3) (layer "F.Cu") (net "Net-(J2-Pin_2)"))
 (segment (start 113.35 117.86) (end 112.95 118.26) (width 0.3) (layer "F.Cu") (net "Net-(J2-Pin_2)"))
 (segment (start 111.95 117.16) (end 109.85 115.06) (width 0.3) (layer "F.Cu") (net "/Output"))
 (segment (start 109.85 111.425) (end 109.925 111.35) (width 0.3) (layer "F.Cu") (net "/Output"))
 (segment (start 109.81054 121.66) (end 109.85 121.66) (width 0.3) (layer "F.Cu") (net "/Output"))
 (segment (start 104.95054 116.8) (end 109.81054 121.66) (width 0.3) (layer "F.Cu") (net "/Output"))
 (segment (start 111.95 119.56) (end 111.95 117.16) (width 0.3) (layer "F.Cu") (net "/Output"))
 (segment (start 109.85 115.06) (end 109.85 111.425) (width 0.3) (layer "F.Cu") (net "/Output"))
 (segment (start 109.85 121.66) (end 111.95 119.56) (width 0.3) (layer "F.Cu") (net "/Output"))
 (segment (start 103.80054 115.41) (end 103.80054 125.45054) (width 0.3) (layer "F.Cu") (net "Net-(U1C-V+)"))
 (segment (start 109 128.2) (end 106.55 128.2) (width 0.3) (layer "F.Cu") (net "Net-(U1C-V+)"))
 (segment (start 114.5 133.7) (end 109 128.2) (width 0.3) (layer "F.Cu") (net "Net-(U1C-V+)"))
 (segment (start 103.80054 125.45054) (end 106.55 128.2) (width 0.3) (layer "F.Cu") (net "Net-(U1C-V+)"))
 (segment (start 104.95054 114.26) (end 103.80054 115.41) (width 0.3) (layer "F.Cu") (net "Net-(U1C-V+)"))
 (segment (start 114.5 134.2) (end 114.5 133.7) (width 0.3) (layer "F.Cu") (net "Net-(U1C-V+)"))
 (segment (start 117 115.32) (end 113.21 115.32) (width 0.3) (layer "F.Cu") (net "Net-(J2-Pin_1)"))
 (segment (start 113.21 115.32) (end 112.95 115.06) (width 0.3) (layer "F.Cu") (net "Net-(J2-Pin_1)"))
 (segment (start 114.21 120.4) (end 112.95 121.66) (width 0.3) (layer "F.Cu") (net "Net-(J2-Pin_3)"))
 (segment (start 117 120.4) (end 114.21 120.4) (width 0.3) (layer "F.Cu") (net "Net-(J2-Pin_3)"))
 (segment (start 101.63554 101.086262) (end 101.63554 100.6) (width 0.3) (layer "F.Cu") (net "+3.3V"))
 (segment (start 101.14804 104.3) (end 101.14804 101.573762) (width 0.3) (layer "F.Cu") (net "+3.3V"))
 (segment (start 101.14804 101.573762) (end 101.63554 101.086262) (width 0.3) (layer "F.Cu") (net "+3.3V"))
 (segment (start 100.64804 100.6125) (end 100.63554 100.6) (width 0.3) (layer "F.Cu") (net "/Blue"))
 (segment (start 100.64804 104.3) (end 100.64804 100.6125) (width 0.3) (layer "F.Cu") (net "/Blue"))
 (segment (start 99.63554 103.7875) (end 99.63554 100.6) (width 0.3) (layer "F.Cu") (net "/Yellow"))
 (segment (start 100.14804 104.3) (end 99.63554 103.7875) (width 0.3) (layer "F.Cu") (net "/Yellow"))
 (segment (start 103.45 128.2) (end 103.45 130.275) (width 0.3) (layer "F.Cu") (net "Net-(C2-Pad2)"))
 (segment (start 103.775 130.6) (end 103.6 130.425) (width 0.3) (layer "F.Cu") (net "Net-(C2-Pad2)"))
 (segment (start 106.6 130.6) (end 103.775 130.6) (width 0.3) (layer "F.Cu") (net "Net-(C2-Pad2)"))
 (segment (start 103.45 130.275) (end 103.6 130.425) (width 0.3) (layer "F.Cu") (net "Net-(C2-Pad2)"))
 (segment (start 109.275 107.05) (end 109.275 106.398762) (width 0.3) (layer "F.Cu") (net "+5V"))
 (segment (start 104.1 105.9) (end 106.567894 108.367894) (width 0.3) (layer "F.Cu") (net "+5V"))
 (segment (start 109.275 108.125) (end 109.275 107.05) (width 0.3) (layer "F.Cu") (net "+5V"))
 (segment (start 109.275 106.398762) (end 110.5 105.173762) (width 0.3) (layer "F.Cu") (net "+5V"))
 (segment (start 87.175 105.9) (end 104.1 105.9) (width 0.3) (layer "F.Cu") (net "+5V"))
 (segment (start 106.567894 108.367894) (end 109.032106 108.367894) (width 0.3) (layer "F.Cu") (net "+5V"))
 (segment (start 110.5 105.173762) (end 110.5 102.8) (width 0.3) (layer "F.Cu") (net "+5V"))
 (segment (start 87.2 103.4) (end 87.2 105.875) (width 0.3) (layer "F.Cu") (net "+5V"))
 (segment (start 109.032106 108.367894) (end 109.275 108.125) (width 0.3) (layer "F.Cu") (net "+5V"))
 (segment (start 87.2 105.875) (end 87.175 105.9) (width 0.3) (layer "F.Cu") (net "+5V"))
 (segment (start 108.625 107.05) (end 108.625 102.825) (width 0.3) (layer "F.Cu") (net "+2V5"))
 (segment (start 108.625 102.825) (end 108.6 102.8) (width 0.3) (layer "F.Cu") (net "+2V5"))
 (segment (start 109.925 107.05) (end 110.575 107.05) (width 0.3) (layer "F.Cu") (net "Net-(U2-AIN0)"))
 (segment (start 101.64804 109.55196) (end 101.64804 108.6) (width 0.3) (layer "F.Cu") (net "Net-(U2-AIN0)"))
 (segment (start 109.825 107.15) (end 109.825 108.575) (width 0.3) (layer "F.Cu") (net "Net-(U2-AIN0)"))
 (segment (start 109.825 108.575) (end 108.725 109.675) (width 0.3) (layer "F.Cu") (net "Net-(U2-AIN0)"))
 (segment (start 101.77108 109.675) (end 101.64804 109.55196) (width 0.3) (layer "F.Cu") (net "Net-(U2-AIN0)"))
 (segment (start 108.725 109.675) (end 101.77108 109.675) (width 0.3) (layer "F.Cu") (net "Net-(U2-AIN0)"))
 (segment (start 109.925 107.05) (end 109.825 107.15) (width 0.3) (layer "F.Cu") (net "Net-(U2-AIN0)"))
 (segment (start 98.8 130.425) (end 98.8 128.35) (width 0.3) (layer "F.Cu") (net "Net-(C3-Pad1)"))
 (segment (start 96.3 130.425) (end 96.2 130.525) (width 0.3) (layer "F.Cu") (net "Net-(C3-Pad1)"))
 (segment (start 98.8 128.35) (end 98.95 128.2) (width 0.3) (layer "F.Cu") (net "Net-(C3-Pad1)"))
 (segment (start 98.8 130.425) (end 96.3 130.425) (width 0.3) (layer "F.Cu") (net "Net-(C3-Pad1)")))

